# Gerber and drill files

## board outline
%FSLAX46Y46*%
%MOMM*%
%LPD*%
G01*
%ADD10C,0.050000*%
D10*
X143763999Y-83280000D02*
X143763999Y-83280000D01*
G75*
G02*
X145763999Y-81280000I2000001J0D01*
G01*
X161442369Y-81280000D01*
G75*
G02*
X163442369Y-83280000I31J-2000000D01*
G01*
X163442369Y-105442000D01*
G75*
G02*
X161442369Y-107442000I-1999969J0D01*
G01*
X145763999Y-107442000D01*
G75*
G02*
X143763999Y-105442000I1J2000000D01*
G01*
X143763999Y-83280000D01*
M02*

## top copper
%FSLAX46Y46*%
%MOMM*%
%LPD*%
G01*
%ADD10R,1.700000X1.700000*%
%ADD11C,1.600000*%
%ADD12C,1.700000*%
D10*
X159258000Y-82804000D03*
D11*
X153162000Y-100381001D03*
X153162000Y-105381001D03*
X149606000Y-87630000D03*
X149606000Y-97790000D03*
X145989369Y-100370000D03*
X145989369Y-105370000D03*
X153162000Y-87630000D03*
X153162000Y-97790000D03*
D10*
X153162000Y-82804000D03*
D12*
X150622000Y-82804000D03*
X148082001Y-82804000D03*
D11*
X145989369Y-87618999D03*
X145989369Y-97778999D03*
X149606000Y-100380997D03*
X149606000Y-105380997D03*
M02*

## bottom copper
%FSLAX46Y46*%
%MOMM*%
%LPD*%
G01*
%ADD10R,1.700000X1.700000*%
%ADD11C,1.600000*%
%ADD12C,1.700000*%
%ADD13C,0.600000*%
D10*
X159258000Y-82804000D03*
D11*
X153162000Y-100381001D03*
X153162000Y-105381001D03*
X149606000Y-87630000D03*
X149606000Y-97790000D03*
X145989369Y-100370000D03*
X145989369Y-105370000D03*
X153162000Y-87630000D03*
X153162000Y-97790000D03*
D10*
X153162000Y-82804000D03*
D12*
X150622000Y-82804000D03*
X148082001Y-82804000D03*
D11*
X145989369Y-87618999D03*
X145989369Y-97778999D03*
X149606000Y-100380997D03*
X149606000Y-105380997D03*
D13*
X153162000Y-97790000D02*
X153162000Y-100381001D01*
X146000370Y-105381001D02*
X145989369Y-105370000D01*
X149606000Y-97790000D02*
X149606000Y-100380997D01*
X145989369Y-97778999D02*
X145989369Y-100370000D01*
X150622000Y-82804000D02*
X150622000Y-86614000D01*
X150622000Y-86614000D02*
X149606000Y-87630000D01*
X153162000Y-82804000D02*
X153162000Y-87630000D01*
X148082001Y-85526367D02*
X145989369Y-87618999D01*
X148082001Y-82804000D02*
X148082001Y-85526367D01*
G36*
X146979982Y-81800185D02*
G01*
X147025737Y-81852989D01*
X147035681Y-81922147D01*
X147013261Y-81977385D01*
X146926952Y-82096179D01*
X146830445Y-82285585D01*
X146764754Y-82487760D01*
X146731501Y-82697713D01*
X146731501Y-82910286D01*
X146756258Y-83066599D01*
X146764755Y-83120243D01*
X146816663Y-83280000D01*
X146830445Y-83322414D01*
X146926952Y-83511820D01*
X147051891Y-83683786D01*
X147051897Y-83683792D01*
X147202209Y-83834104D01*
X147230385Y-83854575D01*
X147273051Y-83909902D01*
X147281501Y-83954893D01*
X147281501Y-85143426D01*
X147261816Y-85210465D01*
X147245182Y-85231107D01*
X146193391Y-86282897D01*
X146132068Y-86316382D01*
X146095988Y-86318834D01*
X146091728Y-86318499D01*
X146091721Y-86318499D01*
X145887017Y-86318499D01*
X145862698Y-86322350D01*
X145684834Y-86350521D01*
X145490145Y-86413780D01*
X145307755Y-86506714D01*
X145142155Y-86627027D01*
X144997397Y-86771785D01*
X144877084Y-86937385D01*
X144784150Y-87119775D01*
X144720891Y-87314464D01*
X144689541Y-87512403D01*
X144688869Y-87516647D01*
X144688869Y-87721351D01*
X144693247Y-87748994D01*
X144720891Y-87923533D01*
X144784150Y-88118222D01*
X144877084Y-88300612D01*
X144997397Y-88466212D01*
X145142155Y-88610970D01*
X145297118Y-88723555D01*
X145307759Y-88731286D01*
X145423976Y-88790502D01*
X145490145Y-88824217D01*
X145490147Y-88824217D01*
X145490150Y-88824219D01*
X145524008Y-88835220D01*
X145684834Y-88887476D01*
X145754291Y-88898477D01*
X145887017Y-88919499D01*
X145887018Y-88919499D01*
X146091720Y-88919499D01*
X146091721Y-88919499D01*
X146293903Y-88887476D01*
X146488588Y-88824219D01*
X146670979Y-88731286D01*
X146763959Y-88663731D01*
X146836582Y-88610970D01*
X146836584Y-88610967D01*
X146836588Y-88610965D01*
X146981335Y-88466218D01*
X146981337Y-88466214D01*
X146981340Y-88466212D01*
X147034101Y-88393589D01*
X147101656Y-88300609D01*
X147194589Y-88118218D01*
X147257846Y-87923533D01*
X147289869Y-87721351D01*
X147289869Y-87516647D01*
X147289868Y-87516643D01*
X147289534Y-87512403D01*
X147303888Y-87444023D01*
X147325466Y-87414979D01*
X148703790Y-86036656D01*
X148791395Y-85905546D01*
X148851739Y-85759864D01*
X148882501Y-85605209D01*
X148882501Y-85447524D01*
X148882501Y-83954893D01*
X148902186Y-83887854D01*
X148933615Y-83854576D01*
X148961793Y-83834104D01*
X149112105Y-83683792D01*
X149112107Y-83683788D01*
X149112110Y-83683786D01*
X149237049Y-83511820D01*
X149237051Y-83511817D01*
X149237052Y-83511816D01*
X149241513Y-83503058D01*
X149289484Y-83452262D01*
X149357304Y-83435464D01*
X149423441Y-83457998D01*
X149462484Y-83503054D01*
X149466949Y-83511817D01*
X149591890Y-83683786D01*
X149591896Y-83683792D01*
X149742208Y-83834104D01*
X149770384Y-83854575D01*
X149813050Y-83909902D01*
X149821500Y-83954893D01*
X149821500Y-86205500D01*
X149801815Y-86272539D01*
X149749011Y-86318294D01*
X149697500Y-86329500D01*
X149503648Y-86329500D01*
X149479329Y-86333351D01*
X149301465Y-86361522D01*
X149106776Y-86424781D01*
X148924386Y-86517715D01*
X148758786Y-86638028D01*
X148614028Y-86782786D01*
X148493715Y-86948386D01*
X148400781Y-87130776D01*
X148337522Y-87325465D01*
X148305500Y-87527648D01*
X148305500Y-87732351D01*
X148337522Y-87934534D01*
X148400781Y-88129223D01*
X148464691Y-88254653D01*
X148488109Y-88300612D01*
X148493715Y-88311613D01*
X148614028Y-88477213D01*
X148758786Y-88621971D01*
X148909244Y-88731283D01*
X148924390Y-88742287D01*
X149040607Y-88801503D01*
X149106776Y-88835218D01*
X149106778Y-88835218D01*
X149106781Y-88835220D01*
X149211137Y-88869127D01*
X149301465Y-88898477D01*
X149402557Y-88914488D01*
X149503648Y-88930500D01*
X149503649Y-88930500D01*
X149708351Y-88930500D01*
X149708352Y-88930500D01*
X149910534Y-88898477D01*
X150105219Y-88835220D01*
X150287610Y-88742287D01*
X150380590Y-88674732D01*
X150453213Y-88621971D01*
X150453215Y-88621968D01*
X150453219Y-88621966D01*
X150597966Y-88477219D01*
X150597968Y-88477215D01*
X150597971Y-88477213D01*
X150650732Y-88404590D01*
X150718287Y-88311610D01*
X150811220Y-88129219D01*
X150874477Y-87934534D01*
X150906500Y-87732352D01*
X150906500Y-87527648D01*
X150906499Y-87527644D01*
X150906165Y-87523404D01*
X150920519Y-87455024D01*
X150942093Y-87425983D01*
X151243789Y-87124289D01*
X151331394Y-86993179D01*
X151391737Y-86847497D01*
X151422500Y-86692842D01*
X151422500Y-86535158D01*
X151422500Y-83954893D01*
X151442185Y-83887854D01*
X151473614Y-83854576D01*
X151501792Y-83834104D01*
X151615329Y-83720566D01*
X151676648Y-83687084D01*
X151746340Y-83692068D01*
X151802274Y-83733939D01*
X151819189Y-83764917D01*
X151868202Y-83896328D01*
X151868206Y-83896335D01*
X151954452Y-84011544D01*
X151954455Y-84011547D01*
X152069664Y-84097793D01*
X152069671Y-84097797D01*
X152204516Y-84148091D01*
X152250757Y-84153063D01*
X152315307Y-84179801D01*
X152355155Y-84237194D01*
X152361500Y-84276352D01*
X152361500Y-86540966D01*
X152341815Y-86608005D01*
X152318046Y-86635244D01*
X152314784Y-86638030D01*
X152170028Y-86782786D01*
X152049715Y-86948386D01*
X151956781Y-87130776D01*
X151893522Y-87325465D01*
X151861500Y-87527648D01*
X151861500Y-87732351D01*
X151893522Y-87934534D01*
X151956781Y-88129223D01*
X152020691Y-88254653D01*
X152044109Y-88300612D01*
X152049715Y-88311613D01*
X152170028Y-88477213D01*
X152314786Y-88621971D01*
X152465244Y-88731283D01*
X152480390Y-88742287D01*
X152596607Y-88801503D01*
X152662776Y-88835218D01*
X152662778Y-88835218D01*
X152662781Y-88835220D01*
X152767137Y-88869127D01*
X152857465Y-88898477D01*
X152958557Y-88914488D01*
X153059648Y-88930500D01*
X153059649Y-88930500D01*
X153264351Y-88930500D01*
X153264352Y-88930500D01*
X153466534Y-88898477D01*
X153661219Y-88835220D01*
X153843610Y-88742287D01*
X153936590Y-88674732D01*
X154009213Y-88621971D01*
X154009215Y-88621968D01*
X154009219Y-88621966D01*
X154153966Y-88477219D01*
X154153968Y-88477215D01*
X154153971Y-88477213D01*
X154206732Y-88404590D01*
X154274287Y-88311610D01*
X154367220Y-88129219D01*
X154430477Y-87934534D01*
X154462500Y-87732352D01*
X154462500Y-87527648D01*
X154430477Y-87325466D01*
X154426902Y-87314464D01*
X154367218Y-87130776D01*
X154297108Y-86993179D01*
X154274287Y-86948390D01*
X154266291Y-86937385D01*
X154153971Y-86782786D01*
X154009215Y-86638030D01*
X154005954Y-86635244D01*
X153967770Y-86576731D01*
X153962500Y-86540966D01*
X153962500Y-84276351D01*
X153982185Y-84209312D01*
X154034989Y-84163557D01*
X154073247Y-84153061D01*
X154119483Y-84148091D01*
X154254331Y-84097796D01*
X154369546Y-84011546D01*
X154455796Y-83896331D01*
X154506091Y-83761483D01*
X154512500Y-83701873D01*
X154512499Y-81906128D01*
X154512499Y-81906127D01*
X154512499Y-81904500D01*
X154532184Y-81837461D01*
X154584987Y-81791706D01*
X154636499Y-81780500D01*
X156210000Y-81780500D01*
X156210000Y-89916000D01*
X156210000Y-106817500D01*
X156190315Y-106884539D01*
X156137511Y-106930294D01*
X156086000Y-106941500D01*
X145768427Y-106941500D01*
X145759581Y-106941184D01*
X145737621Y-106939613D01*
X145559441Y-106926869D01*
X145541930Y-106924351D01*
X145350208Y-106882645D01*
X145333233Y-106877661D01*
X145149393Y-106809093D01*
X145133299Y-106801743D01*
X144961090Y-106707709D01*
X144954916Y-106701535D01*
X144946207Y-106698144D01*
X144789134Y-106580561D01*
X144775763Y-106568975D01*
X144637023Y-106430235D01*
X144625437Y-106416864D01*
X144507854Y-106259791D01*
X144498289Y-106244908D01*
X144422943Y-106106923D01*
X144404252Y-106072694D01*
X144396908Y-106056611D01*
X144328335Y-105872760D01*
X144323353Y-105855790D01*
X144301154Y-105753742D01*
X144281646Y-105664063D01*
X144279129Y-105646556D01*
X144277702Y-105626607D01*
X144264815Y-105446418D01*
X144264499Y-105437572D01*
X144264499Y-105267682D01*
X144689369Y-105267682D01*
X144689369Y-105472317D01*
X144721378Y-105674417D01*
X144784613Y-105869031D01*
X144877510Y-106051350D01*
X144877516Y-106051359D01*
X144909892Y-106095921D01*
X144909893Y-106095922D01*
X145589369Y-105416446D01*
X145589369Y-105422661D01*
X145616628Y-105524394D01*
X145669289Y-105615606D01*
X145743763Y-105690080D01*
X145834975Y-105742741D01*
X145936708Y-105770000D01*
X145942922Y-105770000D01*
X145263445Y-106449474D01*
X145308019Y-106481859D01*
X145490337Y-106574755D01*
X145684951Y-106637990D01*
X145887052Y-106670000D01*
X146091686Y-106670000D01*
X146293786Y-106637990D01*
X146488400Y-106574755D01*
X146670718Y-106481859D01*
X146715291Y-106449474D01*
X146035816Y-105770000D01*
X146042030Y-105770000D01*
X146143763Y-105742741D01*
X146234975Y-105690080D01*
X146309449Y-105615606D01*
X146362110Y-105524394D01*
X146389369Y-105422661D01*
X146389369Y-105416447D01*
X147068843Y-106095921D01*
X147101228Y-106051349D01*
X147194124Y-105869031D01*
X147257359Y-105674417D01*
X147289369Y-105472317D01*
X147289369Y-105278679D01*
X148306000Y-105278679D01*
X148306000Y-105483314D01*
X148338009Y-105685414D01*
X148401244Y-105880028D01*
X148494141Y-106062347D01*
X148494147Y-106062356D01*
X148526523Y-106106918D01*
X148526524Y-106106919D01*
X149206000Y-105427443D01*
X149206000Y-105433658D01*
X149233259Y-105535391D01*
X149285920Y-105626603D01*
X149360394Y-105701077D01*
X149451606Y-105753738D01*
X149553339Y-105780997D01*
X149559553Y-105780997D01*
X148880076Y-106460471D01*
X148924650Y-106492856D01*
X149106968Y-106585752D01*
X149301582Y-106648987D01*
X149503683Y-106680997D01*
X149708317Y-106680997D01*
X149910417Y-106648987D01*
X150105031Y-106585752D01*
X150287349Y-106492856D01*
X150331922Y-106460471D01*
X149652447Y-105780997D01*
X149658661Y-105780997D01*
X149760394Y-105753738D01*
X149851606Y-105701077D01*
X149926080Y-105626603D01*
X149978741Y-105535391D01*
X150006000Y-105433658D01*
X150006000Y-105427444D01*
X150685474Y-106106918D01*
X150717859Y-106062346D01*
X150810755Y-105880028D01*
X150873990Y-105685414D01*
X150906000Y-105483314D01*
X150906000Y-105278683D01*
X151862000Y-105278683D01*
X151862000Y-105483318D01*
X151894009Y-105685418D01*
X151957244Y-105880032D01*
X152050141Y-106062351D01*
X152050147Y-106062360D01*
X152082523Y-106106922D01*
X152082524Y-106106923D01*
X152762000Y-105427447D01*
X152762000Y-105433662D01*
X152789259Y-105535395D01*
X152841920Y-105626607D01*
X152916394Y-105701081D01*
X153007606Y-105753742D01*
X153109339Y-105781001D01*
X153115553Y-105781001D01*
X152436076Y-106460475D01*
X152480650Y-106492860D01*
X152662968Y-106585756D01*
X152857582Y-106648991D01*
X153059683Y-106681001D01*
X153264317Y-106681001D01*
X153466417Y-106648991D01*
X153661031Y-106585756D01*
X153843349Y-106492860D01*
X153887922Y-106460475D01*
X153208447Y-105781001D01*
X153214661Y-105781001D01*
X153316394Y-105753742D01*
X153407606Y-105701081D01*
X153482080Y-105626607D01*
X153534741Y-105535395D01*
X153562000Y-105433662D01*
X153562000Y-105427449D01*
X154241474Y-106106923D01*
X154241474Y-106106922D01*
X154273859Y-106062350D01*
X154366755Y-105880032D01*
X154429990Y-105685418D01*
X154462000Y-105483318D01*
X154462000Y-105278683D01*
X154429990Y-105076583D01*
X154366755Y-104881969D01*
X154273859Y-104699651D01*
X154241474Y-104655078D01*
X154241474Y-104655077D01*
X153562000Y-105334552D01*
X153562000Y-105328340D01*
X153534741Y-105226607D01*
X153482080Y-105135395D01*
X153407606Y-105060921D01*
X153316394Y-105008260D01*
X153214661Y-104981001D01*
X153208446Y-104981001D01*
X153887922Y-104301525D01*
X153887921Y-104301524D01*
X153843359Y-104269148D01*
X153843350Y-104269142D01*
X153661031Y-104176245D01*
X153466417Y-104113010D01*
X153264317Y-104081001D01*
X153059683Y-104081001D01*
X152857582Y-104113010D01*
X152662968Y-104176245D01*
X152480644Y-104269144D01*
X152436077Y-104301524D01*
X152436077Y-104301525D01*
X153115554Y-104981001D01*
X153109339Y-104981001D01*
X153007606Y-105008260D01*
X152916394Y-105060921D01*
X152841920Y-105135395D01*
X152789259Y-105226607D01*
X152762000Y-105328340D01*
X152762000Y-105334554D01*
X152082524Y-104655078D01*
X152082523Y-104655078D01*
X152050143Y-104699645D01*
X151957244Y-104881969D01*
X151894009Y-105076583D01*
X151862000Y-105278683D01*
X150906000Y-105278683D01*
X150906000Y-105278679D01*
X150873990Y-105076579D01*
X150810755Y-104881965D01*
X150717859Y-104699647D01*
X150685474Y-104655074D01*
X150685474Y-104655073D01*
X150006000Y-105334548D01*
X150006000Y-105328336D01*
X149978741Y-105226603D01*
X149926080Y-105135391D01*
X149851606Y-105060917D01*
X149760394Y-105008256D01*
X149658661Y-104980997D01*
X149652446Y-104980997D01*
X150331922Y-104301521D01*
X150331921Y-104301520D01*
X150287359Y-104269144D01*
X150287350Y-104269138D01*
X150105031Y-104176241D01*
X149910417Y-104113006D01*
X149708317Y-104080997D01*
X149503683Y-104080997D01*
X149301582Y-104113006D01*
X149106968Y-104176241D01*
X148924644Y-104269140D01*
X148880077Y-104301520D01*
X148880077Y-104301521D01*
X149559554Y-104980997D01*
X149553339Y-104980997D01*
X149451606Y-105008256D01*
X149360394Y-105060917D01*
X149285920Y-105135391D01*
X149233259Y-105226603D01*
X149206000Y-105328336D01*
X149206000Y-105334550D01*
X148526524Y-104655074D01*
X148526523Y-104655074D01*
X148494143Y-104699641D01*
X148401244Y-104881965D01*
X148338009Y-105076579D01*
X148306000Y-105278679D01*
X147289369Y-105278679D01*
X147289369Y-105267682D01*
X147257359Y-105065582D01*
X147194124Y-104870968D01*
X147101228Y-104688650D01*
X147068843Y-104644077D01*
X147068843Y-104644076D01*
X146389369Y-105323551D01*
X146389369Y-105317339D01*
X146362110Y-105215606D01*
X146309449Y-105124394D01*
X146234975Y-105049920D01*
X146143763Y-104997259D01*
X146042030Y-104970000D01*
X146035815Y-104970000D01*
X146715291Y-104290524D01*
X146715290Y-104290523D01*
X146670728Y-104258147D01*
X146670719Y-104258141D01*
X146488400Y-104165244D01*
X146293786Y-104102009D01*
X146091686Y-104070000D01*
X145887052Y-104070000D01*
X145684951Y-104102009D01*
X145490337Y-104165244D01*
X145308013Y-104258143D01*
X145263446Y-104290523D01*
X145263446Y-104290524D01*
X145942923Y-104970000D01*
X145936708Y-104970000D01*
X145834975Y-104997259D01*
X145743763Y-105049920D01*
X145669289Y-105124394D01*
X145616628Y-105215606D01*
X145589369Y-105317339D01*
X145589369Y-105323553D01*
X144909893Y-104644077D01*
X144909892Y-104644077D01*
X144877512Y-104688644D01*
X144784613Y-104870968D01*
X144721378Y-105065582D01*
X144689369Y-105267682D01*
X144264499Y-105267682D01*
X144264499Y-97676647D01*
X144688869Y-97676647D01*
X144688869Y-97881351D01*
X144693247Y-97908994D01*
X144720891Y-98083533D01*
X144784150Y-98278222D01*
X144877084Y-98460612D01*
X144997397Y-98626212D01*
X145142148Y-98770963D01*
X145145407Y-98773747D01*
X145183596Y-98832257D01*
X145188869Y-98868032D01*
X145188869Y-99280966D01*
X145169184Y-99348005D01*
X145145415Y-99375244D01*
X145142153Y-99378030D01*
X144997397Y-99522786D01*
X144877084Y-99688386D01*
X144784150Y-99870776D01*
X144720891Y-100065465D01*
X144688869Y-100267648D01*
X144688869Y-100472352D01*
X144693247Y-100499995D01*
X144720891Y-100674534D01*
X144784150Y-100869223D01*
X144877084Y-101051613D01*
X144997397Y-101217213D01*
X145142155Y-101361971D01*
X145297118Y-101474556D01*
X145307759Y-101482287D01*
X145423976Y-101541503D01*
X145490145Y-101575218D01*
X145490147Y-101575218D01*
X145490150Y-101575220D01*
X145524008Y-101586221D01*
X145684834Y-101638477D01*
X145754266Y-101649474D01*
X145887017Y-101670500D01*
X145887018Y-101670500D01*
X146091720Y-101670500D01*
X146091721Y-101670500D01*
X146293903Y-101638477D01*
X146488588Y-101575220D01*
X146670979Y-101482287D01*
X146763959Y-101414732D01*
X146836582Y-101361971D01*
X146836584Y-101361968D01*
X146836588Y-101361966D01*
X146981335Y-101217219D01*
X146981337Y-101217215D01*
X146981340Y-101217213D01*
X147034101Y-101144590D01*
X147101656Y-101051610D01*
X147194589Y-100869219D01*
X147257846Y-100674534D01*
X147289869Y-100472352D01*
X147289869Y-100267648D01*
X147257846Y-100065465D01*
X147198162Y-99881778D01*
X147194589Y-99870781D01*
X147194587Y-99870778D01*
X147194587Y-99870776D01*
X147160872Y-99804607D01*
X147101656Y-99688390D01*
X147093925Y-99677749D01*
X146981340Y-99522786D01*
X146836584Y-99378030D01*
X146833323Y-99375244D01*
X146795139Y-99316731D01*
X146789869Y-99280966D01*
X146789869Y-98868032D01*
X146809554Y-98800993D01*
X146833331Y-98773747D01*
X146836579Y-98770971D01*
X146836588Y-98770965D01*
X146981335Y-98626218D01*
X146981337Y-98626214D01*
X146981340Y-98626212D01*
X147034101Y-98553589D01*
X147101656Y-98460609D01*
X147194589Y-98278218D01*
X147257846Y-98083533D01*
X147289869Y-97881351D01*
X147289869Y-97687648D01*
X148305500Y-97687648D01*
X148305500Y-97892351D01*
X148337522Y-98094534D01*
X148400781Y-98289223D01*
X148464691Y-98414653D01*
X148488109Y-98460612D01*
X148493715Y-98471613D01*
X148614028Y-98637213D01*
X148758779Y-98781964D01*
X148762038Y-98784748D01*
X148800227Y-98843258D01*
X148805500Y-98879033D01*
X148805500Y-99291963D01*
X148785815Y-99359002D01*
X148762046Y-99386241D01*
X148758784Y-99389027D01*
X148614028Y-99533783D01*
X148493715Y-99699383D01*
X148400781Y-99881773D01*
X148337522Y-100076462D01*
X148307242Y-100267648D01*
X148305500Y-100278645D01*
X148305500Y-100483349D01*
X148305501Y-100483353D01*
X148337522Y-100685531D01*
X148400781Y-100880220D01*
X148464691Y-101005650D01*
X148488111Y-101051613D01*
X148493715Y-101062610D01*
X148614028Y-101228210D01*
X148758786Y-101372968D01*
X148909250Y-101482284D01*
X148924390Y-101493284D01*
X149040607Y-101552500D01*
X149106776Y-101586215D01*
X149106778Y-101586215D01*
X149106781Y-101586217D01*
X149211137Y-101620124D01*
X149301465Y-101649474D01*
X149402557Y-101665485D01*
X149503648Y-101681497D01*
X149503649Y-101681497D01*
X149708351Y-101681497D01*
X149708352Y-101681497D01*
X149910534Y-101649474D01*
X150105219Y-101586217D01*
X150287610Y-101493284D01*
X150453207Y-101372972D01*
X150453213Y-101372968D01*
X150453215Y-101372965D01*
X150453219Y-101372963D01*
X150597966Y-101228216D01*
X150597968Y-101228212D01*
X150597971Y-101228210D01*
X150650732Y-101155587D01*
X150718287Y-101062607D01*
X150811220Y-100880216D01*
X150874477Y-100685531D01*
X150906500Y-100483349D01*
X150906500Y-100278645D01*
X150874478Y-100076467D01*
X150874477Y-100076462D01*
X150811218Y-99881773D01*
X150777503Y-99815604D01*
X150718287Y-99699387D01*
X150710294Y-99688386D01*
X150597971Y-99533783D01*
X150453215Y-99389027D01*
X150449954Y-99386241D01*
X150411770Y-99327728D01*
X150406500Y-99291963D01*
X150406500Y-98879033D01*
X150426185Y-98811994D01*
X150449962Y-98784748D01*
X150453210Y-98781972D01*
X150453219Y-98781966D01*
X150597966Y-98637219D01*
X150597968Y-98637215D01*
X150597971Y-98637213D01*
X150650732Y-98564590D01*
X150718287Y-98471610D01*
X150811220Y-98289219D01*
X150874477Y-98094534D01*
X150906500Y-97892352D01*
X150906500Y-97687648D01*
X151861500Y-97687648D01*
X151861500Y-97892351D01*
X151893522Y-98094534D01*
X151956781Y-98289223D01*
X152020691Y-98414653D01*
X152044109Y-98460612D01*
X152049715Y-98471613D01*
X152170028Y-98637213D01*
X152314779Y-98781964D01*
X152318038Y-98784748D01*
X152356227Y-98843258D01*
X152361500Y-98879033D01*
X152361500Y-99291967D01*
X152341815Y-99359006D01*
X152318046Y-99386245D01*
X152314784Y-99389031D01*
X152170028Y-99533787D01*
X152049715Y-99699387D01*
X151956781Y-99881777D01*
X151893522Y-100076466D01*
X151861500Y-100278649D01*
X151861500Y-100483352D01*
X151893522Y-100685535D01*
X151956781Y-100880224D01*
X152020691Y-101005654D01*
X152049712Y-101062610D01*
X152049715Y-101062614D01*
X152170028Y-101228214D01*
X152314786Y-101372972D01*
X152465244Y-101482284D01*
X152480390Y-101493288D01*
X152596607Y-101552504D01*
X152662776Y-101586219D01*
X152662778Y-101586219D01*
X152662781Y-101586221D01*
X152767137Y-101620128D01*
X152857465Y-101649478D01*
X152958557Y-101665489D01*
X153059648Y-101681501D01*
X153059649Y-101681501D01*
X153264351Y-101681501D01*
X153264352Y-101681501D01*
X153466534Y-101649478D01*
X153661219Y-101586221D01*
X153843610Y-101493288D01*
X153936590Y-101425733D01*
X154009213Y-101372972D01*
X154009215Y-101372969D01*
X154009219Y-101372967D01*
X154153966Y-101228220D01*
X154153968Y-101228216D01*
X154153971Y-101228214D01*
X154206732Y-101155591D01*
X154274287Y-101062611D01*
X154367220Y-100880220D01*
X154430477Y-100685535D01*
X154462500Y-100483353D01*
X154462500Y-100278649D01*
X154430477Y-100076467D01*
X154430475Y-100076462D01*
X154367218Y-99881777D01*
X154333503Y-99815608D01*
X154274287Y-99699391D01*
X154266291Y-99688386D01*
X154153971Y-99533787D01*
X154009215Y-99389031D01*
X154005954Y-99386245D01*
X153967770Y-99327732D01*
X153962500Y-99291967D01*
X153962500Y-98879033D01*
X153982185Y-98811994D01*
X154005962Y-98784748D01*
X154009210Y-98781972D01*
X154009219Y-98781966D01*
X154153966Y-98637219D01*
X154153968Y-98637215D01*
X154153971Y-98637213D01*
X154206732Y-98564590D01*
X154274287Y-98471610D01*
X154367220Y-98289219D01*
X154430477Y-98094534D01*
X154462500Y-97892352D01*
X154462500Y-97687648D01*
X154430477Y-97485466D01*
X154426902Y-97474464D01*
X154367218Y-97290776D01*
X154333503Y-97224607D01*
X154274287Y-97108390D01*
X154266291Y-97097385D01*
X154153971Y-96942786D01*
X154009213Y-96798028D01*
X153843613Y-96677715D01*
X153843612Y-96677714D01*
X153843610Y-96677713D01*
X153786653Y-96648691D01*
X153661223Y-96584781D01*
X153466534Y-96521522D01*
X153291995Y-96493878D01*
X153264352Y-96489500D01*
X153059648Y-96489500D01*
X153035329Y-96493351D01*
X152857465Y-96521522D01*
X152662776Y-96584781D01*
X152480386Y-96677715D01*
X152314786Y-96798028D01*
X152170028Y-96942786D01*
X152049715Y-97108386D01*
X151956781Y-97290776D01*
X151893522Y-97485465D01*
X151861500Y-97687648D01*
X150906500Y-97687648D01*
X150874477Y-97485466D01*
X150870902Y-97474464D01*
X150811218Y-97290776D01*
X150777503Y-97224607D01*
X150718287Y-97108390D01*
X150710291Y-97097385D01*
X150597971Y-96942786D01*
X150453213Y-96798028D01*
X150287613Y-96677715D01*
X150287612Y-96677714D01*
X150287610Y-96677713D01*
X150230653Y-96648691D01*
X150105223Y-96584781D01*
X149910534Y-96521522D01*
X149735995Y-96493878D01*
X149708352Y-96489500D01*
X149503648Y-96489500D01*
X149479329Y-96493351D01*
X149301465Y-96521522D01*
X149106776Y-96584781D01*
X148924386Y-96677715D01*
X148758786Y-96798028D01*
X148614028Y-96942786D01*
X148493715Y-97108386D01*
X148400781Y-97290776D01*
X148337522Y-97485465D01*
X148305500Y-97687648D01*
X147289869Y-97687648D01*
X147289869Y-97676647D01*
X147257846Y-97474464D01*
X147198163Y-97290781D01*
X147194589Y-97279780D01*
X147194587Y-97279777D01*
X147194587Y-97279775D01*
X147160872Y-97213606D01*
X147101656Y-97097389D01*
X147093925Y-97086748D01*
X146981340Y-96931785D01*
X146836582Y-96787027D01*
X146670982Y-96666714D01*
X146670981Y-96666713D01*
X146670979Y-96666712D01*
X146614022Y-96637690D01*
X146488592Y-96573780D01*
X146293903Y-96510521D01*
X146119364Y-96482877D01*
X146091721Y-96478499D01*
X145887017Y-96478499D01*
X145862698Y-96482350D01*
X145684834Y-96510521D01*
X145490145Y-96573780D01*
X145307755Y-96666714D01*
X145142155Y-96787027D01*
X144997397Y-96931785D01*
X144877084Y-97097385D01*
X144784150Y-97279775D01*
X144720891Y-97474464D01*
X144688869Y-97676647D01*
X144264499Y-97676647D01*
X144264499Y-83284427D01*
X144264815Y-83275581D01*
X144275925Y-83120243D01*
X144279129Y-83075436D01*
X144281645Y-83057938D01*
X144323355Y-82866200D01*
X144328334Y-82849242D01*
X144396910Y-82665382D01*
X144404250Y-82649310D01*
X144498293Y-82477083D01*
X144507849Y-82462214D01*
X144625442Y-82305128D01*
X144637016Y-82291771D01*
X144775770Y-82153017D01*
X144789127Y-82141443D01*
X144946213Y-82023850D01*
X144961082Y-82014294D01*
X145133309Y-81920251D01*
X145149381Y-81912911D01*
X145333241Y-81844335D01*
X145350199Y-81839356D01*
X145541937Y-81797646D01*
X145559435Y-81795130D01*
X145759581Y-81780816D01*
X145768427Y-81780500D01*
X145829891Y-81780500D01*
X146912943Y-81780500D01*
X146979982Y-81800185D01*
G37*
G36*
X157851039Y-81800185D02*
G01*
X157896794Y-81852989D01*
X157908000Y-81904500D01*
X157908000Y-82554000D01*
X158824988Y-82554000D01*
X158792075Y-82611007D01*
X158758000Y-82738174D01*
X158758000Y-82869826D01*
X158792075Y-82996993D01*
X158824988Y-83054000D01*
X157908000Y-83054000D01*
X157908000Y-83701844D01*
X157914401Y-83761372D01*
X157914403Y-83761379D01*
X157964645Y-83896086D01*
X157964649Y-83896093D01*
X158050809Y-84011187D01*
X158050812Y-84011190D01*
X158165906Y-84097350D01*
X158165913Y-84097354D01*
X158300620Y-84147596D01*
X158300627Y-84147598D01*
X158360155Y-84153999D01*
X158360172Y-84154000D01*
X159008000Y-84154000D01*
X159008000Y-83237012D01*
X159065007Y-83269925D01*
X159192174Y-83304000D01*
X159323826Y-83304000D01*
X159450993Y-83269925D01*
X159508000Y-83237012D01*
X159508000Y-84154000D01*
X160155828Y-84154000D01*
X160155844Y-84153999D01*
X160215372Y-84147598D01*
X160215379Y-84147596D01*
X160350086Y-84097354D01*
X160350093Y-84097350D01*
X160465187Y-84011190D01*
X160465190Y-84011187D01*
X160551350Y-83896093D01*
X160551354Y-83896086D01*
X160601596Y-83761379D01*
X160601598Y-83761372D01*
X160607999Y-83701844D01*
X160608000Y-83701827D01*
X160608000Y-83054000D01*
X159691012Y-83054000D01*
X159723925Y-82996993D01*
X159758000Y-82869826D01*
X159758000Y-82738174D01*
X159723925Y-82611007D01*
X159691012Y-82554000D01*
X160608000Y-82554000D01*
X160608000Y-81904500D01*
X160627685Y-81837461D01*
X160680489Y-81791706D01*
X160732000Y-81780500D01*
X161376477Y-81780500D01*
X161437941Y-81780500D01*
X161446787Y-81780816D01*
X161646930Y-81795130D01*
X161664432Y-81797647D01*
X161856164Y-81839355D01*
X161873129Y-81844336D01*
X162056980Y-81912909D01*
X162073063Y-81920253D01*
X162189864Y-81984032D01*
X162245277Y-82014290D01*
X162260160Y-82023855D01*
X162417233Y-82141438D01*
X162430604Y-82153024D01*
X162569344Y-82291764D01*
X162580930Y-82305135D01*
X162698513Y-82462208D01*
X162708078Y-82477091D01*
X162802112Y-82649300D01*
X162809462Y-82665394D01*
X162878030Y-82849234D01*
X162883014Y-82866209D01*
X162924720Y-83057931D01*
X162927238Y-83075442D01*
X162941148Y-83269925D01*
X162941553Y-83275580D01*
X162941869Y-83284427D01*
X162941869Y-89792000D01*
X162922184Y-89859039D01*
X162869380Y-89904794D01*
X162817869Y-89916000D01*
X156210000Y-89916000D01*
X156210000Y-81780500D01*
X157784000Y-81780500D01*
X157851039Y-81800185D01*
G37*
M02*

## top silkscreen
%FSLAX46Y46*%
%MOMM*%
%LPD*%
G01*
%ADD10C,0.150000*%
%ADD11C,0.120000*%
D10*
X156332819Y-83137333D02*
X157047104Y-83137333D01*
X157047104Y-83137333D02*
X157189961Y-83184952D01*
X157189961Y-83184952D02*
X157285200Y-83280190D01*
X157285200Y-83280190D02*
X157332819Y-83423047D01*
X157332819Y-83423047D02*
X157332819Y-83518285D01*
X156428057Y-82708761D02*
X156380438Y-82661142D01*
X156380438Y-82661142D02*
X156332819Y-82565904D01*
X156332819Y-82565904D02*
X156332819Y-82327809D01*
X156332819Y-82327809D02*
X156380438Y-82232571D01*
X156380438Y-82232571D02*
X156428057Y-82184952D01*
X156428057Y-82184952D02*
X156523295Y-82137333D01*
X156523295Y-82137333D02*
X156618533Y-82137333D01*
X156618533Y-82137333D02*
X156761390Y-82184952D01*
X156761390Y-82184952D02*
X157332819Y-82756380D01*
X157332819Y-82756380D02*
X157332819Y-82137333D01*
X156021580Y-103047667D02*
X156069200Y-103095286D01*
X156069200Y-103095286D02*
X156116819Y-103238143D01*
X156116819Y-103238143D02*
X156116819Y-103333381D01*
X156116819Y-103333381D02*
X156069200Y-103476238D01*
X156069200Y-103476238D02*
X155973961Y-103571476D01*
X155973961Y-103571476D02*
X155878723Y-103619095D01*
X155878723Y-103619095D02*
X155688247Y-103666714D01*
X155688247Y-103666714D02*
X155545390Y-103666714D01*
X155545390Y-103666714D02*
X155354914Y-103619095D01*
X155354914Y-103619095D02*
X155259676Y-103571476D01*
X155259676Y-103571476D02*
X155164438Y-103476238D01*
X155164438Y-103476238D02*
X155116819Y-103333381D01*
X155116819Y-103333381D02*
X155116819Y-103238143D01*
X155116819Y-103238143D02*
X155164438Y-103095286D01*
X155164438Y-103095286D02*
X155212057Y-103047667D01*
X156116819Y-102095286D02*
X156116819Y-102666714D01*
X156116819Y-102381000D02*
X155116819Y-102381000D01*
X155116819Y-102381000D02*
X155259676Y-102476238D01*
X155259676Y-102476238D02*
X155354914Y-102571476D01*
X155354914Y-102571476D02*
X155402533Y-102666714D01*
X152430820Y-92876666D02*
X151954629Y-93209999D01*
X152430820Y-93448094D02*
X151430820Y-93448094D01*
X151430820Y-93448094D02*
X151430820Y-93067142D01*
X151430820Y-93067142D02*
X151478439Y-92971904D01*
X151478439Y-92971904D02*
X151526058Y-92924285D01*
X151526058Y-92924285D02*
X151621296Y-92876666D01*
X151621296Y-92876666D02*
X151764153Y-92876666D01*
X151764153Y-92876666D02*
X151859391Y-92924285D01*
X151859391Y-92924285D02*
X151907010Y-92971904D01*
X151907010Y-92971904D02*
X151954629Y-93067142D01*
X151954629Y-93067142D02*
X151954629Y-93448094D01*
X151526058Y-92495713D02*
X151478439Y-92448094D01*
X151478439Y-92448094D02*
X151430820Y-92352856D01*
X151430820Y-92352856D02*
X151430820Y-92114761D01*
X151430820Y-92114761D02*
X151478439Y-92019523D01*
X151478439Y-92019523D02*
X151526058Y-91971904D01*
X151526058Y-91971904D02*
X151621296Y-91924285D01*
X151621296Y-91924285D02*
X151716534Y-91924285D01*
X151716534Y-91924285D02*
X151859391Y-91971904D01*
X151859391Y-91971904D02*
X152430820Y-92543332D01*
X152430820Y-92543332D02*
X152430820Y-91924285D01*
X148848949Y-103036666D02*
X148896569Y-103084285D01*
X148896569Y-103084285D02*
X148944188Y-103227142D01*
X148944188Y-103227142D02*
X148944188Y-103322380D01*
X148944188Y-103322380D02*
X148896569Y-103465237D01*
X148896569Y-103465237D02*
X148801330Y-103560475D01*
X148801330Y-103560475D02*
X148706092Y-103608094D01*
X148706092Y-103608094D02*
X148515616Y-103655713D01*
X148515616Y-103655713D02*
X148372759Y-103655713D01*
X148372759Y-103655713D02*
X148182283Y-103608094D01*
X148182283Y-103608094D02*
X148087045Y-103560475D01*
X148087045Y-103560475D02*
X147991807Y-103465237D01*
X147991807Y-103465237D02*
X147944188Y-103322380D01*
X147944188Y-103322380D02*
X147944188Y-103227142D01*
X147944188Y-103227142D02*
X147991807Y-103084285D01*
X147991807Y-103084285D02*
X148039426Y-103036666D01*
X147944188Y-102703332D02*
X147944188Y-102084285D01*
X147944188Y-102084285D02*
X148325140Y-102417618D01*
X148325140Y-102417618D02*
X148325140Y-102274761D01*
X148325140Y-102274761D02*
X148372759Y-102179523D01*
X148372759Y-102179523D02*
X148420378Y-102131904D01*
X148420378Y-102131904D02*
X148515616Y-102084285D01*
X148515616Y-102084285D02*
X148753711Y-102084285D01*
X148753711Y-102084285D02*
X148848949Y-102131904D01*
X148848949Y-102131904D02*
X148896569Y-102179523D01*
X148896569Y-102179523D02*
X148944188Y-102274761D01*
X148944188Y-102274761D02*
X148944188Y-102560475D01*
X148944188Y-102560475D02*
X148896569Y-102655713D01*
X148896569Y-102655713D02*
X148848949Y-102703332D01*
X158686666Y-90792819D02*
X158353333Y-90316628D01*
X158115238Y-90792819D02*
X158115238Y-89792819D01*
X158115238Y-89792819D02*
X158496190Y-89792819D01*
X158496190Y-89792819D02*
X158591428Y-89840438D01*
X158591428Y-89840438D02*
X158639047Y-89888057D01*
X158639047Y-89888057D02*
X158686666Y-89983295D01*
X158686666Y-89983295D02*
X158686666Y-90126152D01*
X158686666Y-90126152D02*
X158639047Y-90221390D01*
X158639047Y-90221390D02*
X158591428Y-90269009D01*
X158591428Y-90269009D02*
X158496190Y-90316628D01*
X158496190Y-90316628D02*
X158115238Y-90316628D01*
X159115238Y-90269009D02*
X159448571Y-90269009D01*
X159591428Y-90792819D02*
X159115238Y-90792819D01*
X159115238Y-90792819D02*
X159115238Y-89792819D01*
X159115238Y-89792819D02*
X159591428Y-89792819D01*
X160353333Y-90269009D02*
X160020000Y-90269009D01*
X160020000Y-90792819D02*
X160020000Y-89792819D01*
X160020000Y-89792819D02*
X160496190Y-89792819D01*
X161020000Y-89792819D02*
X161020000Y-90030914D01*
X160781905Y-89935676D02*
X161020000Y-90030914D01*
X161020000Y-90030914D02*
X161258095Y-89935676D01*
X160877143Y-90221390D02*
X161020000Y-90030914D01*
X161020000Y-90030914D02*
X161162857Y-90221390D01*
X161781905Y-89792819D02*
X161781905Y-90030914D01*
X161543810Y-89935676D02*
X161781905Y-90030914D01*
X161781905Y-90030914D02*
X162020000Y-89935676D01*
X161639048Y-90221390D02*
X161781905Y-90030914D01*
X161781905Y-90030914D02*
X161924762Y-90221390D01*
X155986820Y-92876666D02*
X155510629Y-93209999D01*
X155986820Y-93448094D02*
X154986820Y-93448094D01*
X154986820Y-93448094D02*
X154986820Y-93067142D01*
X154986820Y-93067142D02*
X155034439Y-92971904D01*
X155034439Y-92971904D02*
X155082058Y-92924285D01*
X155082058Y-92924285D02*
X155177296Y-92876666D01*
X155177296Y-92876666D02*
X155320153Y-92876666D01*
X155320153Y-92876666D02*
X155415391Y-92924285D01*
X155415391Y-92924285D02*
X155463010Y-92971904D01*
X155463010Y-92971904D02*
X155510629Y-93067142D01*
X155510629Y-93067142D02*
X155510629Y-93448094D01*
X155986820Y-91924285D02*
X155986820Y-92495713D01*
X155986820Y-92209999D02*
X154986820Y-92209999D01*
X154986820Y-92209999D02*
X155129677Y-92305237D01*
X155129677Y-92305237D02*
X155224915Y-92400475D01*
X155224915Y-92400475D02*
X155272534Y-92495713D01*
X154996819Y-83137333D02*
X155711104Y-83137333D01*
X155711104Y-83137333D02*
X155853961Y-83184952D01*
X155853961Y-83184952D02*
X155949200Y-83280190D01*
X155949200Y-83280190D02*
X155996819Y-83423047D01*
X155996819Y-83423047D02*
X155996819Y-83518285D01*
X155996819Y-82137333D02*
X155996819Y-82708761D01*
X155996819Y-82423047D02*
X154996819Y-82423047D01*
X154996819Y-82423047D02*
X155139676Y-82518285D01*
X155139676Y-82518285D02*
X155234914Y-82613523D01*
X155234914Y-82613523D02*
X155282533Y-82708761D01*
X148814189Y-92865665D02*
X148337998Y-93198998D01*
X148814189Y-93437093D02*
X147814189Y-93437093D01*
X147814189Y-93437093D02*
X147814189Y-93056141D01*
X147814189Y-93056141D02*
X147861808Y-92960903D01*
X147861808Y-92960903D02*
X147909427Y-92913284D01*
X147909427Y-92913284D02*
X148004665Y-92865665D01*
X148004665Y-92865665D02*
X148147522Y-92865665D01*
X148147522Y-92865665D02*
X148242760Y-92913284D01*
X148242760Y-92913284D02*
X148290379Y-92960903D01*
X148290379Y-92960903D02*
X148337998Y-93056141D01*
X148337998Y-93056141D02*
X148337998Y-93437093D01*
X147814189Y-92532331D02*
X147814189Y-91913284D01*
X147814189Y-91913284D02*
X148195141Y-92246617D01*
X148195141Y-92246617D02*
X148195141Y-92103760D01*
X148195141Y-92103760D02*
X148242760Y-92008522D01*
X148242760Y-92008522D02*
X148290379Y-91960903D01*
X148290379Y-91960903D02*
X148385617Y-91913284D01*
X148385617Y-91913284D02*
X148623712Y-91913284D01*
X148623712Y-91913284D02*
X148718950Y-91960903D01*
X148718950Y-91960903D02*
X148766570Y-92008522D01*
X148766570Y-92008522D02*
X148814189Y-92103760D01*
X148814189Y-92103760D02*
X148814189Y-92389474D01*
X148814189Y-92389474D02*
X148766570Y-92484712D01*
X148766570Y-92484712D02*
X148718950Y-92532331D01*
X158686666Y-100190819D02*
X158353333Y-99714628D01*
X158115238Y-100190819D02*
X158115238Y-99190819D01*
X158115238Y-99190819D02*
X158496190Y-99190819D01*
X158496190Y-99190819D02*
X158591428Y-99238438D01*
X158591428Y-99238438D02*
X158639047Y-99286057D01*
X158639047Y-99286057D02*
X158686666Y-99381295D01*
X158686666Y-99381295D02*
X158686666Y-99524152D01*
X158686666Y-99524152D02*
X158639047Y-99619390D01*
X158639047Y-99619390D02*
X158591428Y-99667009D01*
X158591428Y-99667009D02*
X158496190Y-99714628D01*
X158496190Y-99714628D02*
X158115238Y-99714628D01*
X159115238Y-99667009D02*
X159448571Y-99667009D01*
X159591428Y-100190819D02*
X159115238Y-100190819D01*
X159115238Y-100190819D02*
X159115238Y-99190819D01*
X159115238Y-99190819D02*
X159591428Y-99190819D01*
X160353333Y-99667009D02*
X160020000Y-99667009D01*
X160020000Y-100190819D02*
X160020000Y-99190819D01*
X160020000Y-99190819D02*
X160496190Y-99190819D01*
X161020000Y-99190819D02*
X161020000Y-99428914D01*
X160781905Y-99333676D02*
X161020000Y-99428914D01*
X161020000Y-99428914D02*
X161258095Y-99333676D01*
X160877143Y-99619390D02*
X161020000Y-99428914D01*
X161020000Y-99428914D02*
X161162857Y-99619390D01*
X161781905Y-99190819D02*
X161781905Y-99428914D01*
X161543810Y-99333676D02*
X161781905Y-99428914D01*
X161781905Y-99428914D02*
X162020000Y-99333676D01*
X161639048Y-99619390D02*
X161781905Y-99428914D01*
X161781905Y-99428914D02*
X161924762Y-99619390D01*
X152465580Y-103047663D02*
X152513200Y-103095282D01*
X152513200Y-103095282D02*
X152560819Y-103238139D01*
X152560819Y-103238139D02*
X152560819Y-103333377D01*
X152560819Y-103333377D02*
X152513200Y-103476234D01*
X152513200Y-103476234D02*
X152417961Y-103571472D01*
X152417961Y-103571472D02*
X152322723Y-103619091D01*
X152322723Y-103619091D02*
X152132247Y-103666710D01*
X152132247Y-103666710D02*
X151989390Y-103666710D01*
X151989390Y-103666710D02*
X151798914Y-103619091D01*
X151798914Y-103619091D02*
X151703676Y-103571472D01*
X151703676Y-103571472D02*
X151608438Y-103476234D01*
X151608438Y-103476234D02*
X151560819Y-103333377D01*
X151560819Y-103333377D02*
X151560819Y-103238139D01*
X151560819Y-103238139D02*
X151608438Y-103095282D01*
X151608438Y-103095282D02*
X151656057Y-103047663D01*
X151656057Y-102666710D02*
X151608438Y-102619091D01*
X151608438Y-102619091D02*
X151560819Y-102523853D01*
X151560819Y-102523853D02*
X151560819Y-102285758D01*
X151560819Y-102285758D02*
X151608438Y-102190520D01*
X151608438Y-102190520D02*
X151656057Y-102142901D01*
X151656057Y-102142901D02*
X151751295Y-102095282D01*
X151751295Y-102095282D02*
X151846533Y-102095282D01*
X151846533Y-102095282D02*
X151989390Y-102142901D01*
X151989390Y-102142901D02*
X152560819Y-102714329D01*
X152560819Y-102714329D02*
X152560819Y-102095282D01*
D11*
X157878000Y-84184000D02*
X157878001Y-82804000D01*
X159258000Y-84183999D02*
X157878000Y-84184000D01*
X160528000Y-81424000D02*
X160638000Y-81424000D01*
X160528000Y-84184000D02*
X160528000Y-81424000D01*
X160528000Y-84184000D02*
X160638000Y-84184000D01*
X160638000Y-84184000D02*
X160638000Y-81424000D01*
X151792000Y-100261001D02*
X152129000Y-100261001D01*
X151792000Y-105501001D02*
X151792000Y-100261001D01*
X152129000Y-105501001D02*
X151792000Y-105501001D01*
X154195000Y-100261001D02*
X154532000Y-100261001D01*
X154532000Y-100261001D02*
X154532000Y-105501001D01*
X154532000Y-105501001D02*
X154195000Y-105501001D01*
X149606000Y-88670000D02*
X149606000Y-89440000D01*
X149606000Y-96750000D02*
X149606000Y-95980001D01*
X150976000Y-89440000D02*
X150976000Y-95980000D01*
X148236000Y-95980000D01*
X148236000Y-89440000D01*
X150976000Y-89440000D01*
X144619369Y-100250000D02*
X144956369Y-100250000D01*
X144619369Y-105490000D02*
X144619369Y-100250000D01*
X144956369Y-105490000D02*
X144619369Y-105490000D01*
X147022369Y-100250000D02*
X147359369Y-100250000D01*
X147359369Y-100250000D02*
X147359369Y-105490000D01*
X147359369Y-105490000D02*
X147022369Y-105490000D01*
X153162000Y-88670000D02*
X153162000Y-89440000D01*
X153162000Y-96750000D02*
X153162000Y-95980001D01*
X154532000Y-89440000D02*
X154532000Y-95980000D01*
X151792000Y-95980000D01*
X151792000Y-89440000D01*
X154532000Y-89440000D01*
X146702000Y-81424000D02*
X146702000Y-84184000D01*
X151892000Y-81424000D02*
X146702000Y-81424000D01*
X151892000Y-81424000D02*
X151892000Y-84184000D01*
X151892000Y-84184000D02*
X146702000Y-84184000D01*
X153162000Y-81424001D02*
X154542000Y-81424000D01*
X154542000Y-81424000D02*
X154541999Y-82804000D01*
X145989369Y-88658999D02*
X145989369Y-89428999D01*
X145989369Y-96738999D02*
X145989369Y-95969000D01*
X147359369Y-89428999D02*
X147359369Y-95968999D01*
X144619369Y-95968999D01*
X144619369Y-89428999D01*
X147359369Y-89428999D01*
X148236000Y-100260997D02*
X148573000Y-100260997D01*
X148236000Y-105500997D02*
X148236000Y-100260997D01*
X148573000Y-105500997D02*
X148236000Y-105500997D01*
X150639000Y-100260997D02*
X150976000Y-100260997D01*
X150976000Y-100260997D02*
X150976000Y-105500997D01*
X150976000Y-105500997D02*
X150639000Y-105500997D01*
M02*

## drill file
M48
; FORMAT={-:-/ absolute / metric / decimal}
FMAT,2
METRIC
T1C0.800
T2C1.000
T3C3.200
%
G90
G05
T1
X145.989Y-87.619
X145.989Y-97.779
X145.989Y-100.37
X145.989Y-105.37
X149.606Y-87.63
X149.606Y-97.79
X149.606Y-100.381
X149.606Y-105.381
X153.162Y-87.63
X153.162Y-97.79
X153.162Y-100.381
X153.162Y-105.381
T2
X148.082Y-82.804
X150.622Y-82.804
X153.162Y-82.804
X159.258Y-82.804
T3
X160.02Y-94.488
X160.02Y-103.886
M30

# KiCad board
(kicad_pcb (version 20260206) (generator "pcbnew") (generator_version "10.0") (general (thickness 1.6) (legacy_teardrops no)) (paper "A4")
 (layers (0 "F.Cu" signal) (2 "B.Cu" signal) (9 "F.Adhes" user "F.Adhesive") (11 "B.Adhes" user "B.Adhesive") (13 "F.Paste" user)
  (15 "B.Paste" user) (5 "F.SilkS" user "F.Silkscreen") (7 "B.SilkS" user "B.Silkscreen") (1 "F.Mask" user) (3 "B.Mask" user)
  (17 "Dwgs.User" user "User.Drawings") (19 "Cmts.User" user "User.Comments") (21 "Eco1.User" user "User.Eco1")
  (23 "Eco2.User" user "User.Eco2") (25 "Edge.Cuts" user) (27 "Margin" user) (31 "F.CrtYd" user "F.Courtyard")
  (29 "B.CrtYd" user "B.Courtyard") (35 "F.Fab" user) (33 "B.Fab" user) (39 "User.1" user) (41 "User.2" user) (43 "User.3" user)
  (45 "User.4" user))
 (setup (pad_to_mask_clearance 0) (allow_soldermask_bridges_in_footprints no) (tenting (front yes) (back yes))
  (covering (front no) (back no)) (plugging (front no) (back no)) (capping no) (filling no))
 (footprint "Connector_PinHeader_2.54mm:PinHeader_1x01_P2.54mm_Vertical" (layer "F.Cu") (at 159.258 82.804 90)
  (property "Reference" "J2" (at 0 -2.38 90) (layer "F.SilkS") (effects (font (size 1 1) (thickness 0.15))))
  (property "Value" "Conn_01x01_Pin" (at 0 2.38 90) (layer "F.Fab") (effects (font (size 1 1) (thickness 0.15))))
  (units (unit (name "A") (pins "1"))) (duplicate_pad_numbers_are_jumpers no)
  (fp_line (start -1.38 -1.38) (end 0 -1.379999) (stroke (width 0.12) (type solid)) (layer "F.SilkS"))
  (fp_line (start -1.379999 0) (end -1.38 -1.38) (stroke (width 0.12) (type solid)) (layer "F.SilkS"))
  (fp_line (start 1.38 1.27) (end 1.38 1.38) (stroke (width 0.12) (type solid)) (layer "F.SilkS"))
  (fp_line (start -1.38 1.27) (end 1.38 1.27) (stroke (width 0.12) (type solid)) (layer "F.SilkS"))
  (fp_line (start -1.38 1.27) (end -1.38 1.38) (stroke (width 0.12) (type solid)) (layer "F.SilkS"))
  (fp_line (start -1.38 1.38) (end 1.38 1.38) (stroke (width 0.12) (type solid)) (layer "F.SilkS"))
  (pad "1" thru_hole rect (at 0 0 90) (size 1.7 1.7) (drill 1) (layers "*.Cu" "*.Mask") (remove_unused_layers no) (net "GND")))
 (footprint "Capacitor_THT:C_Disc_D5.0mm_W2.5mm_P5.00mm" (layer "F.Cu") (at 153.162 100.381001 -90)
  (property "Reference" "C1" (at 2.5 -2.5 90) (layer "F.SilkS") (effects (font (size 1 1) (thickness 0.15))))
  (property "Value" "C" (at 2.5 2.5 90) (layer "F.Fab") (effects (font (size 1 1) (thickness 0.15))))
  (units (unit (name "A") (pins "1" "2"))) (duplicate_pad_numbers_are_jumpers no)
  (fp_line (start -0.12 1.37) (end -0.12 1.033) (stroke (width 0.12) (type solid)) (layer "F.SilkS"))
  (fp_line (start 5.12 1.37) (end -0.12 1.37) (stroke (width 0.12) (type solid)) (layer "F.SilkS"))
  (fp_line (start 5.12 1.033) (end 5.12 1.37) (stroke (width 0.12) (type solid)) (layer "F.SilkS"))
  (fp_line (start -0.12 -1.033) (end -0.12 -1.37) (stroke (width 0.12) (type solid)) (layer "F.SilkS"))
  (fp_line (start -0.12 -1.37) (end 5.12 -1.37) (stroke (width 0.12) (type solid)) (layer "F.SilkS"))
  (fp_line (start 5.12 -1.37) (end 5.12 -1.033) (stroke (width 0.12) (type solid)) (layer "F.SilkS"))
  (pad "1" thru_hole circle (at 0 0 270) (size 1.6 1.6) (drill 0.8) (layers "*.Cu" "*.Mask") (remove_unused_layers no) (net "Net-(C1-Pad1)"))
  (pad "2" thru_hole circle (at 5 0 270) (size 1.6 1.6) (drill 0.8) (layers "*.Cu" "*.Mask") (remove_unused_layers no) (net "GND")))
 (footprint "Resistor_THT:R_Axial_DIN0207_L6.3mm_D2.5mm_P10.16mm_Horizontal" (layer "F.Cu") (at 149.606 87.63 -90)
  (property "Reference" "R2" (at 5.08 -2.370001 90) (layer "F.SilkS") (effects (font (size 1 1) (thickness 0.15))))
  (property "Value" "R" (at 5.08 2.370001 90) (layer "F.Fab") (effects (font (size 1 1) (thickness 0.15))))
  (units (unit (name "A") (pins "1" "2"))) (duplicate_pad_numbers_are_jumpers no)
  (fp_line (start 1.04 0) (end 1.81 0) (stroke (width 0.12) (type solid)) (layer "F.SilkS"))
  (fp_line (start 9.12 0) (end 8.350001 0) (stroke (width 0.12) (type solid)) (layer "F.SilkS"))
  (fp_poly
   (pts (xy 1.81 -1.37) (xy 8.35 -1.37) (xy 8.35 1.37) (xy 1.81 1.37)) (stroke (width 0.12) (type solid)) (fill no) (layer "F.SilkS"))
  (pad "1" thru_hole circle (at 0 0 270) (size 1.6 1.6) (drill 0.8) (layers "*.Cu" "*.Mask") (remove_unused_layers no)
   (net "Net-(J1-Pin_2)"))
  (pad "2" thru_hole circle (at 10.16 0 270) (size 1.6 1.6) (drill 0.8) (layers "*.Cu" "*.Mask") (remove_unused_layers no)
   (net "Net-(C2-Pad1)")))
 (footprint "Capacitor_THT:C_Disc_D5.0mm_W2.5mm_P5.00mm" (layer "F.Cu") (at 145.989369 100.37 -90)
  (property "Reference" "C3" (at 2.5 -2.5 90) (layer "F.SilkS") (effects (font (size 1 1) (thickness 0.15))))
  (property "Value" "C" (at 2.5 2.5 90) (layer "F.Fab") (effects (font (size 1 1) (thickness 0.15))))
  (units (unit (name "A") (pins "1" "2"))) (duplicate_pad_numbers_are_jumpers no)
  (fp_line (start -0.12 1.37) (end -0.12 1.033) (stroke (width 0.12) (type solid)) (layer "F.SilkS"))
  (fp_line (start 5.12 1.37) (end -0.12 1.37) (stroke (width 0.12) (type solid)) (layer "F.SilkS"))
  (fp_line (start 5.12 1.033) (end 5.12 1.37) (stroke (width 0.12) (type solid)) (layer "F.SilkS"))
  (fp_line (start -0.12 -1.033) (end -0.12 -1.37) (stroke (width 0.12) (type solid)) (layer "F.SilkS"))
  (fp_line (start -0.12 -1.37) (end 5.12 -1.37) (stroke (width 0.12) (type solid)) (layer "F.SilkS"))
  (fp_line (start 5.12 -1.37) (end 5.12 -1.033) (stroke (width 0.12) (type solid)) (layer "F.SilkS"))
  (pad "1" thru_hole circle (at 0 0 270) (size 1.6 1.6) (drill 0.8) (layers "*.Cu" "*.Mask") (remove_unused_layers no) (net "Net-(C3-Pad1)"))
  (pad "2" thru_hole circle (at 5 0 270) (size 1.6 1.6) (drill 0.8) (layers "*.Cu" "*.Mask") (remove_unused_layers no) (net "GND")))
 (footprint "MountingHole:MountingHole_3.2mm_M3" (layer "F.Cu") (at 160.02 94.488)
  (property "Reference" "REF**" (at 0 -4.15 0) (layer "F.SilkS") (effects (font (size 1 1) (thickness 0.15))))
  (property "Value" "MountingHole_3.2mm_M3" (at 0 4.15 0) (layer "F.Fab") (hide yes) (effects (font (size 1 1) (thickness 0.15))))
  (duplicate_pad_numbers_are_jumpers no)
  (pad "" np_thru_hole circle (at 0 0) (size 3.2 3.2) (drill 3.2) (layers "*.Cu" "*.Mask")))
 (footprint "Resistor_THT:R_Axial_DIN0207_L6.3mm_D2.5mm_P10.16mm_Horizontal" (layer "F.Cu") (at 153.162 87.63 -90)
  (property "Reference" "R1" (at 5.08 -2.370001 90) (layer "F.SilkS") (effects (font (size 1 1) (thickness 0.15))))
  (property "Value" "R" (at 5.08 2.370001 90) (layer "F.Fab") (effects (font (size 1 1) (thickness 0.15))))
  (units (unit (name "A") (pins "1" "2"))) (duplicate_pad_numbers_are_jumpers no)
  (fp_line (start 1.04 0) (end 1.81 0) (stroke (width 0.12) (type solid)) (layer "F.SilkS"))
  (fp_line (start 9.12 0) (end 8.350001 0) (stroke (width 0.12) (type solid)) (layer "F.SilkS"))
  (fp_poly
   (pts (xy 1.81 -1.37) (xy 8.35 -1.37) (xy 8.35 1.37) (xy 1.81 1.37)) (stroke (width 0.12) (type solid)) (fill no) (layer "F.SilkS"))
  (pad "1" thru_hole circle (at 0 0 270) (size 1.6 1.6) (drill 0.8) (layers "*.Cu" "*.Mask") (remove_unused_layers no)
   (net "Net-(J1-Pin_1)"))
  (pad "2" thru_hole circle (at 10.16 0 270) (size 1.6 1.6) (drill 0.8) (layers "*.Cu" "*.Mask") (remove_unused_layers no)
   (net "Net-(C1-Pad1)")))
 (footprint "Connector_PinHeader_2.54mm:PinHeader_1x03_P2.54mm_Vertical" (layer "F.Cu") (at 153.162 82.804 -90)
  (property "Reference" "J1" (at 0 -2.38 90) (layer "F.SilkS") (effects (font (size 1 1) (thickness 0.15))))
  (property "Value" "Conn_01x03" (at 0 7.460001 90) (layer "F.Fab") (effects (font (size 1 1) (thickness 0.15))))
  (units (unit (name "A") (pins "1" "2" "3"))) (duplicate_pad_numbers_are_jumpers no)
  (fp_line (start -1.38 6.46) (end 1.38 6.46) (stroke (width 0.12) (type solid)) (layer "F.SilkS"))
  (fp_line (start -1.38 1.27) (end -1.38 6.46) (stroke (width 0.12) (type solid)) (layer "F.SilkS"))
  (fp_line (start -1.38 1.27) (end 1.38 1.27) (stroke (width 0.12) (type solid)) (layer "F.SilkS"))
  (fp_line (start 1.38 1.27) (end 1.38 6.46) (stroke (width 0.12) (type solid)) (layer "F.SilkS"))
  (fp_line (start -1.379999 0) (end -1.38 -1.38) (stroke (width 0.12) (type solid)) (layer "F.SilkS"))
  (fp_line (start -1.38 -1.38) (end 0 -1.379999) (stroke (width 0.12) (type solid)) (layer "F.SilkS"))
  (pad "1" thru_hole rect (at 0 0 270) (size 1.7 1.7) (drill 1) (layers "*.Cu" "*.Mask") (remove_unused_layers no) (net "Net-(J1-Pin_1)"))
  (pad "2" thru_hole circle (at 0 2.54 270) (size 1.7 1.7) (drill 1) (layers "*.Cu" "*.Mask") (remove_unused_layers no)
   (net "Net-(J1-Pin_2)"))
  (pad "3" thru_hole circle (at 0 5.079999 270) (size 1.7 1.7) (drill 1) (layers "*.Cu" "*.Mask") (remove_unused_layers no)
   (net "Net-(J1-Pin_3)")))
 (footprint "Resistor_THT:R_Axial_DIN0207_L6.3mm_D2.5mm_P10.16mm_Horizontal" (layer "F.Cu") (at 145.989369 87.618999 -90)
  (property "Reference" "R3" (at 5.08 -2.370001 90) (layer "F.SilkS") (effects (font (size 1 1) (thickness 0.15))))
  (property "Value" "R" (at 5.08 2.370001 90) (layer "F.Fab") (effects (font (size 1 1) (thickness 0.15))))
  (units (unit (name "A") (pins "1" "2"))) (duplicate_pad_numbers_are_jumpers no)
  (fp_line (start 1.04 0) (end 1.81 0) (stroke (width 0.12) (type solid)) (layer "F.SilkS"))
  (fp_line (start 9.12 0) (end 8.350001 0) (stroke (width 0.12) (type solid)) (layer "F.SilkS"))
  (fp_poly
   (pts (xy 1.81 -1.37) (xy 8.35 -1.37) (xy 8.35 1.37) (xy 1.81 1.37)) (stroke (width 0.12) (type solid)) (fill no) (layer "F.SilkS"))
  (pad "1" thru_hole circle (at 0 0 270) (size 1.6 1.6) (drill 0.8) (layers "*.Cu" "*.Mask") (remove_unused_layers no)
   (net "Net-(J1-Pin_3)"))
  (pad "2" thru_hole circle (at 10.16 0 270) (size 1.6 1.6) (drill 0.8) (layers "*.Cu" "*.Mask") (remove_unused_layers no)
   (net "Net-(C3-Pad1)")))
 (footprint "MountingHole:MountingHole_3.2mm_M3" (layer "F.Cu") (at 160.02 103.886)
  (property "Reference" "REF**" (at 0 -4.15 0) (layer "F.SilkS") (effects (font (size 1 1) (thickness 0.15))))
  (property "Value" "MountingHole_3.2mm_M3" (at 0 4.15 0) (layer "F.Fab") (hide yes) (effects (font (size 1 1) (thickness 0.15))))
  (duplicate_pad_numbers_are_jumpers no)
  (pad "" np_thru_hole circle (at 0 0) (size 3.2 3.2) (drill 3.2) (layers "*.Cu" "*.Mask")))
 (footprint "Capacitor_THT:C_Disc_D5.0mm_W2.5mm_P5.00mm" (layer "F.Cu") (at 149.606 100.380997 -90)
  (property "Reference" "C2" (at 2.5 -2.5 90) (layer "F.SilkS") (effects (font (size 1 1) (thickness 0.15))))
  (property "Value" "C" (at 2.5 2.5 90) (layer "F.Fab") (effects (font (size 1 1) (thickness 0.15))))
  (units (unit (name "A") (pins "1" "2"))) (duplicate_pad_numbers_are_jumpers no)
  (fp_line (start -0.12 1.37) (end -0.12 1.033) (stroke (width 0.12) (type solid)) (layer "F.SilkS"))
  (fp_line (start 5.12 1.37) (end -0.12 1.37) (stroke (width 0.12) (type solid)) (layer "F.SilkS"))
  (fp_line (start 5.12 1.033) (end 5.12 1.37) (stroke (width 0.12) (type solid)) (layer "F.SilkS"))
  (fp_line (start -0.12 -1.033) (end -0.12 -1.37) (stroke (width 0.12) (type solid)) (layer "F.SilkS"))
  (fp_line (start -0.12 -1.37) (end 5.12 -1.37) (stroke (width 0.12) (type solid)) (layer "F.SilkS"))
  (fp_line (start 5.12 -1.37) (end 5.12 -1.033) (stroke (width 0.12) (type solid)) (layer "F.SilkS"))
  (pad "1" thru_hole circle (at 0 0 270) (size 1.6 1.6) (drill 0.8) (layers "*.Cu" "*.Mask") (remove_unused_layers no) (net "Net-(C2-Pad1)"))
  (pad "2" thru_hole circle (at 5 0 270) (size 1.6 1.6) (drill 0.8) (layers "*.Cu" "*.Mask") (remove_unused_layers no) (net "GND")))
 (gr_rect (start 143.763999 81.28) (end 163.442369 107.442) (radius 2) (stroke (width 0.05) (type solid)) (fill no) (layer "Edge.Cuts"))
 (segment (start 153.162 97.79) (end 153.162 100.381001) (width 0.6) (layer "B.Cu") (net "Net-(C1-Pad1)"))
 (segment (start 146.00037 105.381001) (end 145.989369 105.37) (width 0.6) (layer "B.Cu") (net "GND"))
 (segment (start 149.606 97.79) (end 149.606 100.380997) (width 0.6) (layer "B.Cu") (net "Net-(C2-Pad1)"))
 (segment (start 145.989369 97.778999) (end 145.989369 100.37) (width 0.6) (layer "B.Cu") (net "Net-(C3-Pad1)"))
 (segment (start 150.622 82.804) (end 150.622 86.614) (width 0.6) (layer "B.Cu") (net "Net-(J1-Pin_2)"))
 (segment (start 150.622 86.614) (end 149.606 87.63) (width 0.6) (layer "B.Cu") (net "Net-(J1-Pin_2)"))
 (segment (start 153.162 82.804) (end 153.162 87.63) (width 0.6) (layer "B.Cu") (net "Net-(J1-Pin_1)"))
 (segment (start 148.082001 85.526367) (end 145.989369 87.618999) (width 0.6) (layer "B.Cu") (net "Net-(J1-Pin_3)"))
 (segment (start 148.082001 82.804) (end 148.082001 85.526367) (width 0.6) (layer "B.Cu") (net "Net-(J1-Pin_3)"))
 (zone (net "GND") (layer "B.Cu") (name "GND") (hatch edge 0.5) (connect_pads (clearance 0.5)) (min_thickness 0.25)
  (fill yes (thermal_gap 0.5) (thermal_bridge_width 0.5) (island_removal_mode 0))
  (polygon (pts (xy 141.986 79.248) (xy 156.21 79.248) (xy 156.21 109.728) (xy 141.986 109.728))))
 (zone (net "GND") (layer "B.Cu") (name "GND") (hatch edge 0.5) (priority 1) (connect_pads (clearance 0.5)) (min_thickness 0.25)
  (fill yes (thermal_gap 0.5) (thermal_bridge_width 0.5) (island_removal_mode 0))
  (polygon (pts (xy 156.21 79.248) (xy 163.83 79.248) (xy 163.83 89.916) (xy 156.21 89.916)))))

